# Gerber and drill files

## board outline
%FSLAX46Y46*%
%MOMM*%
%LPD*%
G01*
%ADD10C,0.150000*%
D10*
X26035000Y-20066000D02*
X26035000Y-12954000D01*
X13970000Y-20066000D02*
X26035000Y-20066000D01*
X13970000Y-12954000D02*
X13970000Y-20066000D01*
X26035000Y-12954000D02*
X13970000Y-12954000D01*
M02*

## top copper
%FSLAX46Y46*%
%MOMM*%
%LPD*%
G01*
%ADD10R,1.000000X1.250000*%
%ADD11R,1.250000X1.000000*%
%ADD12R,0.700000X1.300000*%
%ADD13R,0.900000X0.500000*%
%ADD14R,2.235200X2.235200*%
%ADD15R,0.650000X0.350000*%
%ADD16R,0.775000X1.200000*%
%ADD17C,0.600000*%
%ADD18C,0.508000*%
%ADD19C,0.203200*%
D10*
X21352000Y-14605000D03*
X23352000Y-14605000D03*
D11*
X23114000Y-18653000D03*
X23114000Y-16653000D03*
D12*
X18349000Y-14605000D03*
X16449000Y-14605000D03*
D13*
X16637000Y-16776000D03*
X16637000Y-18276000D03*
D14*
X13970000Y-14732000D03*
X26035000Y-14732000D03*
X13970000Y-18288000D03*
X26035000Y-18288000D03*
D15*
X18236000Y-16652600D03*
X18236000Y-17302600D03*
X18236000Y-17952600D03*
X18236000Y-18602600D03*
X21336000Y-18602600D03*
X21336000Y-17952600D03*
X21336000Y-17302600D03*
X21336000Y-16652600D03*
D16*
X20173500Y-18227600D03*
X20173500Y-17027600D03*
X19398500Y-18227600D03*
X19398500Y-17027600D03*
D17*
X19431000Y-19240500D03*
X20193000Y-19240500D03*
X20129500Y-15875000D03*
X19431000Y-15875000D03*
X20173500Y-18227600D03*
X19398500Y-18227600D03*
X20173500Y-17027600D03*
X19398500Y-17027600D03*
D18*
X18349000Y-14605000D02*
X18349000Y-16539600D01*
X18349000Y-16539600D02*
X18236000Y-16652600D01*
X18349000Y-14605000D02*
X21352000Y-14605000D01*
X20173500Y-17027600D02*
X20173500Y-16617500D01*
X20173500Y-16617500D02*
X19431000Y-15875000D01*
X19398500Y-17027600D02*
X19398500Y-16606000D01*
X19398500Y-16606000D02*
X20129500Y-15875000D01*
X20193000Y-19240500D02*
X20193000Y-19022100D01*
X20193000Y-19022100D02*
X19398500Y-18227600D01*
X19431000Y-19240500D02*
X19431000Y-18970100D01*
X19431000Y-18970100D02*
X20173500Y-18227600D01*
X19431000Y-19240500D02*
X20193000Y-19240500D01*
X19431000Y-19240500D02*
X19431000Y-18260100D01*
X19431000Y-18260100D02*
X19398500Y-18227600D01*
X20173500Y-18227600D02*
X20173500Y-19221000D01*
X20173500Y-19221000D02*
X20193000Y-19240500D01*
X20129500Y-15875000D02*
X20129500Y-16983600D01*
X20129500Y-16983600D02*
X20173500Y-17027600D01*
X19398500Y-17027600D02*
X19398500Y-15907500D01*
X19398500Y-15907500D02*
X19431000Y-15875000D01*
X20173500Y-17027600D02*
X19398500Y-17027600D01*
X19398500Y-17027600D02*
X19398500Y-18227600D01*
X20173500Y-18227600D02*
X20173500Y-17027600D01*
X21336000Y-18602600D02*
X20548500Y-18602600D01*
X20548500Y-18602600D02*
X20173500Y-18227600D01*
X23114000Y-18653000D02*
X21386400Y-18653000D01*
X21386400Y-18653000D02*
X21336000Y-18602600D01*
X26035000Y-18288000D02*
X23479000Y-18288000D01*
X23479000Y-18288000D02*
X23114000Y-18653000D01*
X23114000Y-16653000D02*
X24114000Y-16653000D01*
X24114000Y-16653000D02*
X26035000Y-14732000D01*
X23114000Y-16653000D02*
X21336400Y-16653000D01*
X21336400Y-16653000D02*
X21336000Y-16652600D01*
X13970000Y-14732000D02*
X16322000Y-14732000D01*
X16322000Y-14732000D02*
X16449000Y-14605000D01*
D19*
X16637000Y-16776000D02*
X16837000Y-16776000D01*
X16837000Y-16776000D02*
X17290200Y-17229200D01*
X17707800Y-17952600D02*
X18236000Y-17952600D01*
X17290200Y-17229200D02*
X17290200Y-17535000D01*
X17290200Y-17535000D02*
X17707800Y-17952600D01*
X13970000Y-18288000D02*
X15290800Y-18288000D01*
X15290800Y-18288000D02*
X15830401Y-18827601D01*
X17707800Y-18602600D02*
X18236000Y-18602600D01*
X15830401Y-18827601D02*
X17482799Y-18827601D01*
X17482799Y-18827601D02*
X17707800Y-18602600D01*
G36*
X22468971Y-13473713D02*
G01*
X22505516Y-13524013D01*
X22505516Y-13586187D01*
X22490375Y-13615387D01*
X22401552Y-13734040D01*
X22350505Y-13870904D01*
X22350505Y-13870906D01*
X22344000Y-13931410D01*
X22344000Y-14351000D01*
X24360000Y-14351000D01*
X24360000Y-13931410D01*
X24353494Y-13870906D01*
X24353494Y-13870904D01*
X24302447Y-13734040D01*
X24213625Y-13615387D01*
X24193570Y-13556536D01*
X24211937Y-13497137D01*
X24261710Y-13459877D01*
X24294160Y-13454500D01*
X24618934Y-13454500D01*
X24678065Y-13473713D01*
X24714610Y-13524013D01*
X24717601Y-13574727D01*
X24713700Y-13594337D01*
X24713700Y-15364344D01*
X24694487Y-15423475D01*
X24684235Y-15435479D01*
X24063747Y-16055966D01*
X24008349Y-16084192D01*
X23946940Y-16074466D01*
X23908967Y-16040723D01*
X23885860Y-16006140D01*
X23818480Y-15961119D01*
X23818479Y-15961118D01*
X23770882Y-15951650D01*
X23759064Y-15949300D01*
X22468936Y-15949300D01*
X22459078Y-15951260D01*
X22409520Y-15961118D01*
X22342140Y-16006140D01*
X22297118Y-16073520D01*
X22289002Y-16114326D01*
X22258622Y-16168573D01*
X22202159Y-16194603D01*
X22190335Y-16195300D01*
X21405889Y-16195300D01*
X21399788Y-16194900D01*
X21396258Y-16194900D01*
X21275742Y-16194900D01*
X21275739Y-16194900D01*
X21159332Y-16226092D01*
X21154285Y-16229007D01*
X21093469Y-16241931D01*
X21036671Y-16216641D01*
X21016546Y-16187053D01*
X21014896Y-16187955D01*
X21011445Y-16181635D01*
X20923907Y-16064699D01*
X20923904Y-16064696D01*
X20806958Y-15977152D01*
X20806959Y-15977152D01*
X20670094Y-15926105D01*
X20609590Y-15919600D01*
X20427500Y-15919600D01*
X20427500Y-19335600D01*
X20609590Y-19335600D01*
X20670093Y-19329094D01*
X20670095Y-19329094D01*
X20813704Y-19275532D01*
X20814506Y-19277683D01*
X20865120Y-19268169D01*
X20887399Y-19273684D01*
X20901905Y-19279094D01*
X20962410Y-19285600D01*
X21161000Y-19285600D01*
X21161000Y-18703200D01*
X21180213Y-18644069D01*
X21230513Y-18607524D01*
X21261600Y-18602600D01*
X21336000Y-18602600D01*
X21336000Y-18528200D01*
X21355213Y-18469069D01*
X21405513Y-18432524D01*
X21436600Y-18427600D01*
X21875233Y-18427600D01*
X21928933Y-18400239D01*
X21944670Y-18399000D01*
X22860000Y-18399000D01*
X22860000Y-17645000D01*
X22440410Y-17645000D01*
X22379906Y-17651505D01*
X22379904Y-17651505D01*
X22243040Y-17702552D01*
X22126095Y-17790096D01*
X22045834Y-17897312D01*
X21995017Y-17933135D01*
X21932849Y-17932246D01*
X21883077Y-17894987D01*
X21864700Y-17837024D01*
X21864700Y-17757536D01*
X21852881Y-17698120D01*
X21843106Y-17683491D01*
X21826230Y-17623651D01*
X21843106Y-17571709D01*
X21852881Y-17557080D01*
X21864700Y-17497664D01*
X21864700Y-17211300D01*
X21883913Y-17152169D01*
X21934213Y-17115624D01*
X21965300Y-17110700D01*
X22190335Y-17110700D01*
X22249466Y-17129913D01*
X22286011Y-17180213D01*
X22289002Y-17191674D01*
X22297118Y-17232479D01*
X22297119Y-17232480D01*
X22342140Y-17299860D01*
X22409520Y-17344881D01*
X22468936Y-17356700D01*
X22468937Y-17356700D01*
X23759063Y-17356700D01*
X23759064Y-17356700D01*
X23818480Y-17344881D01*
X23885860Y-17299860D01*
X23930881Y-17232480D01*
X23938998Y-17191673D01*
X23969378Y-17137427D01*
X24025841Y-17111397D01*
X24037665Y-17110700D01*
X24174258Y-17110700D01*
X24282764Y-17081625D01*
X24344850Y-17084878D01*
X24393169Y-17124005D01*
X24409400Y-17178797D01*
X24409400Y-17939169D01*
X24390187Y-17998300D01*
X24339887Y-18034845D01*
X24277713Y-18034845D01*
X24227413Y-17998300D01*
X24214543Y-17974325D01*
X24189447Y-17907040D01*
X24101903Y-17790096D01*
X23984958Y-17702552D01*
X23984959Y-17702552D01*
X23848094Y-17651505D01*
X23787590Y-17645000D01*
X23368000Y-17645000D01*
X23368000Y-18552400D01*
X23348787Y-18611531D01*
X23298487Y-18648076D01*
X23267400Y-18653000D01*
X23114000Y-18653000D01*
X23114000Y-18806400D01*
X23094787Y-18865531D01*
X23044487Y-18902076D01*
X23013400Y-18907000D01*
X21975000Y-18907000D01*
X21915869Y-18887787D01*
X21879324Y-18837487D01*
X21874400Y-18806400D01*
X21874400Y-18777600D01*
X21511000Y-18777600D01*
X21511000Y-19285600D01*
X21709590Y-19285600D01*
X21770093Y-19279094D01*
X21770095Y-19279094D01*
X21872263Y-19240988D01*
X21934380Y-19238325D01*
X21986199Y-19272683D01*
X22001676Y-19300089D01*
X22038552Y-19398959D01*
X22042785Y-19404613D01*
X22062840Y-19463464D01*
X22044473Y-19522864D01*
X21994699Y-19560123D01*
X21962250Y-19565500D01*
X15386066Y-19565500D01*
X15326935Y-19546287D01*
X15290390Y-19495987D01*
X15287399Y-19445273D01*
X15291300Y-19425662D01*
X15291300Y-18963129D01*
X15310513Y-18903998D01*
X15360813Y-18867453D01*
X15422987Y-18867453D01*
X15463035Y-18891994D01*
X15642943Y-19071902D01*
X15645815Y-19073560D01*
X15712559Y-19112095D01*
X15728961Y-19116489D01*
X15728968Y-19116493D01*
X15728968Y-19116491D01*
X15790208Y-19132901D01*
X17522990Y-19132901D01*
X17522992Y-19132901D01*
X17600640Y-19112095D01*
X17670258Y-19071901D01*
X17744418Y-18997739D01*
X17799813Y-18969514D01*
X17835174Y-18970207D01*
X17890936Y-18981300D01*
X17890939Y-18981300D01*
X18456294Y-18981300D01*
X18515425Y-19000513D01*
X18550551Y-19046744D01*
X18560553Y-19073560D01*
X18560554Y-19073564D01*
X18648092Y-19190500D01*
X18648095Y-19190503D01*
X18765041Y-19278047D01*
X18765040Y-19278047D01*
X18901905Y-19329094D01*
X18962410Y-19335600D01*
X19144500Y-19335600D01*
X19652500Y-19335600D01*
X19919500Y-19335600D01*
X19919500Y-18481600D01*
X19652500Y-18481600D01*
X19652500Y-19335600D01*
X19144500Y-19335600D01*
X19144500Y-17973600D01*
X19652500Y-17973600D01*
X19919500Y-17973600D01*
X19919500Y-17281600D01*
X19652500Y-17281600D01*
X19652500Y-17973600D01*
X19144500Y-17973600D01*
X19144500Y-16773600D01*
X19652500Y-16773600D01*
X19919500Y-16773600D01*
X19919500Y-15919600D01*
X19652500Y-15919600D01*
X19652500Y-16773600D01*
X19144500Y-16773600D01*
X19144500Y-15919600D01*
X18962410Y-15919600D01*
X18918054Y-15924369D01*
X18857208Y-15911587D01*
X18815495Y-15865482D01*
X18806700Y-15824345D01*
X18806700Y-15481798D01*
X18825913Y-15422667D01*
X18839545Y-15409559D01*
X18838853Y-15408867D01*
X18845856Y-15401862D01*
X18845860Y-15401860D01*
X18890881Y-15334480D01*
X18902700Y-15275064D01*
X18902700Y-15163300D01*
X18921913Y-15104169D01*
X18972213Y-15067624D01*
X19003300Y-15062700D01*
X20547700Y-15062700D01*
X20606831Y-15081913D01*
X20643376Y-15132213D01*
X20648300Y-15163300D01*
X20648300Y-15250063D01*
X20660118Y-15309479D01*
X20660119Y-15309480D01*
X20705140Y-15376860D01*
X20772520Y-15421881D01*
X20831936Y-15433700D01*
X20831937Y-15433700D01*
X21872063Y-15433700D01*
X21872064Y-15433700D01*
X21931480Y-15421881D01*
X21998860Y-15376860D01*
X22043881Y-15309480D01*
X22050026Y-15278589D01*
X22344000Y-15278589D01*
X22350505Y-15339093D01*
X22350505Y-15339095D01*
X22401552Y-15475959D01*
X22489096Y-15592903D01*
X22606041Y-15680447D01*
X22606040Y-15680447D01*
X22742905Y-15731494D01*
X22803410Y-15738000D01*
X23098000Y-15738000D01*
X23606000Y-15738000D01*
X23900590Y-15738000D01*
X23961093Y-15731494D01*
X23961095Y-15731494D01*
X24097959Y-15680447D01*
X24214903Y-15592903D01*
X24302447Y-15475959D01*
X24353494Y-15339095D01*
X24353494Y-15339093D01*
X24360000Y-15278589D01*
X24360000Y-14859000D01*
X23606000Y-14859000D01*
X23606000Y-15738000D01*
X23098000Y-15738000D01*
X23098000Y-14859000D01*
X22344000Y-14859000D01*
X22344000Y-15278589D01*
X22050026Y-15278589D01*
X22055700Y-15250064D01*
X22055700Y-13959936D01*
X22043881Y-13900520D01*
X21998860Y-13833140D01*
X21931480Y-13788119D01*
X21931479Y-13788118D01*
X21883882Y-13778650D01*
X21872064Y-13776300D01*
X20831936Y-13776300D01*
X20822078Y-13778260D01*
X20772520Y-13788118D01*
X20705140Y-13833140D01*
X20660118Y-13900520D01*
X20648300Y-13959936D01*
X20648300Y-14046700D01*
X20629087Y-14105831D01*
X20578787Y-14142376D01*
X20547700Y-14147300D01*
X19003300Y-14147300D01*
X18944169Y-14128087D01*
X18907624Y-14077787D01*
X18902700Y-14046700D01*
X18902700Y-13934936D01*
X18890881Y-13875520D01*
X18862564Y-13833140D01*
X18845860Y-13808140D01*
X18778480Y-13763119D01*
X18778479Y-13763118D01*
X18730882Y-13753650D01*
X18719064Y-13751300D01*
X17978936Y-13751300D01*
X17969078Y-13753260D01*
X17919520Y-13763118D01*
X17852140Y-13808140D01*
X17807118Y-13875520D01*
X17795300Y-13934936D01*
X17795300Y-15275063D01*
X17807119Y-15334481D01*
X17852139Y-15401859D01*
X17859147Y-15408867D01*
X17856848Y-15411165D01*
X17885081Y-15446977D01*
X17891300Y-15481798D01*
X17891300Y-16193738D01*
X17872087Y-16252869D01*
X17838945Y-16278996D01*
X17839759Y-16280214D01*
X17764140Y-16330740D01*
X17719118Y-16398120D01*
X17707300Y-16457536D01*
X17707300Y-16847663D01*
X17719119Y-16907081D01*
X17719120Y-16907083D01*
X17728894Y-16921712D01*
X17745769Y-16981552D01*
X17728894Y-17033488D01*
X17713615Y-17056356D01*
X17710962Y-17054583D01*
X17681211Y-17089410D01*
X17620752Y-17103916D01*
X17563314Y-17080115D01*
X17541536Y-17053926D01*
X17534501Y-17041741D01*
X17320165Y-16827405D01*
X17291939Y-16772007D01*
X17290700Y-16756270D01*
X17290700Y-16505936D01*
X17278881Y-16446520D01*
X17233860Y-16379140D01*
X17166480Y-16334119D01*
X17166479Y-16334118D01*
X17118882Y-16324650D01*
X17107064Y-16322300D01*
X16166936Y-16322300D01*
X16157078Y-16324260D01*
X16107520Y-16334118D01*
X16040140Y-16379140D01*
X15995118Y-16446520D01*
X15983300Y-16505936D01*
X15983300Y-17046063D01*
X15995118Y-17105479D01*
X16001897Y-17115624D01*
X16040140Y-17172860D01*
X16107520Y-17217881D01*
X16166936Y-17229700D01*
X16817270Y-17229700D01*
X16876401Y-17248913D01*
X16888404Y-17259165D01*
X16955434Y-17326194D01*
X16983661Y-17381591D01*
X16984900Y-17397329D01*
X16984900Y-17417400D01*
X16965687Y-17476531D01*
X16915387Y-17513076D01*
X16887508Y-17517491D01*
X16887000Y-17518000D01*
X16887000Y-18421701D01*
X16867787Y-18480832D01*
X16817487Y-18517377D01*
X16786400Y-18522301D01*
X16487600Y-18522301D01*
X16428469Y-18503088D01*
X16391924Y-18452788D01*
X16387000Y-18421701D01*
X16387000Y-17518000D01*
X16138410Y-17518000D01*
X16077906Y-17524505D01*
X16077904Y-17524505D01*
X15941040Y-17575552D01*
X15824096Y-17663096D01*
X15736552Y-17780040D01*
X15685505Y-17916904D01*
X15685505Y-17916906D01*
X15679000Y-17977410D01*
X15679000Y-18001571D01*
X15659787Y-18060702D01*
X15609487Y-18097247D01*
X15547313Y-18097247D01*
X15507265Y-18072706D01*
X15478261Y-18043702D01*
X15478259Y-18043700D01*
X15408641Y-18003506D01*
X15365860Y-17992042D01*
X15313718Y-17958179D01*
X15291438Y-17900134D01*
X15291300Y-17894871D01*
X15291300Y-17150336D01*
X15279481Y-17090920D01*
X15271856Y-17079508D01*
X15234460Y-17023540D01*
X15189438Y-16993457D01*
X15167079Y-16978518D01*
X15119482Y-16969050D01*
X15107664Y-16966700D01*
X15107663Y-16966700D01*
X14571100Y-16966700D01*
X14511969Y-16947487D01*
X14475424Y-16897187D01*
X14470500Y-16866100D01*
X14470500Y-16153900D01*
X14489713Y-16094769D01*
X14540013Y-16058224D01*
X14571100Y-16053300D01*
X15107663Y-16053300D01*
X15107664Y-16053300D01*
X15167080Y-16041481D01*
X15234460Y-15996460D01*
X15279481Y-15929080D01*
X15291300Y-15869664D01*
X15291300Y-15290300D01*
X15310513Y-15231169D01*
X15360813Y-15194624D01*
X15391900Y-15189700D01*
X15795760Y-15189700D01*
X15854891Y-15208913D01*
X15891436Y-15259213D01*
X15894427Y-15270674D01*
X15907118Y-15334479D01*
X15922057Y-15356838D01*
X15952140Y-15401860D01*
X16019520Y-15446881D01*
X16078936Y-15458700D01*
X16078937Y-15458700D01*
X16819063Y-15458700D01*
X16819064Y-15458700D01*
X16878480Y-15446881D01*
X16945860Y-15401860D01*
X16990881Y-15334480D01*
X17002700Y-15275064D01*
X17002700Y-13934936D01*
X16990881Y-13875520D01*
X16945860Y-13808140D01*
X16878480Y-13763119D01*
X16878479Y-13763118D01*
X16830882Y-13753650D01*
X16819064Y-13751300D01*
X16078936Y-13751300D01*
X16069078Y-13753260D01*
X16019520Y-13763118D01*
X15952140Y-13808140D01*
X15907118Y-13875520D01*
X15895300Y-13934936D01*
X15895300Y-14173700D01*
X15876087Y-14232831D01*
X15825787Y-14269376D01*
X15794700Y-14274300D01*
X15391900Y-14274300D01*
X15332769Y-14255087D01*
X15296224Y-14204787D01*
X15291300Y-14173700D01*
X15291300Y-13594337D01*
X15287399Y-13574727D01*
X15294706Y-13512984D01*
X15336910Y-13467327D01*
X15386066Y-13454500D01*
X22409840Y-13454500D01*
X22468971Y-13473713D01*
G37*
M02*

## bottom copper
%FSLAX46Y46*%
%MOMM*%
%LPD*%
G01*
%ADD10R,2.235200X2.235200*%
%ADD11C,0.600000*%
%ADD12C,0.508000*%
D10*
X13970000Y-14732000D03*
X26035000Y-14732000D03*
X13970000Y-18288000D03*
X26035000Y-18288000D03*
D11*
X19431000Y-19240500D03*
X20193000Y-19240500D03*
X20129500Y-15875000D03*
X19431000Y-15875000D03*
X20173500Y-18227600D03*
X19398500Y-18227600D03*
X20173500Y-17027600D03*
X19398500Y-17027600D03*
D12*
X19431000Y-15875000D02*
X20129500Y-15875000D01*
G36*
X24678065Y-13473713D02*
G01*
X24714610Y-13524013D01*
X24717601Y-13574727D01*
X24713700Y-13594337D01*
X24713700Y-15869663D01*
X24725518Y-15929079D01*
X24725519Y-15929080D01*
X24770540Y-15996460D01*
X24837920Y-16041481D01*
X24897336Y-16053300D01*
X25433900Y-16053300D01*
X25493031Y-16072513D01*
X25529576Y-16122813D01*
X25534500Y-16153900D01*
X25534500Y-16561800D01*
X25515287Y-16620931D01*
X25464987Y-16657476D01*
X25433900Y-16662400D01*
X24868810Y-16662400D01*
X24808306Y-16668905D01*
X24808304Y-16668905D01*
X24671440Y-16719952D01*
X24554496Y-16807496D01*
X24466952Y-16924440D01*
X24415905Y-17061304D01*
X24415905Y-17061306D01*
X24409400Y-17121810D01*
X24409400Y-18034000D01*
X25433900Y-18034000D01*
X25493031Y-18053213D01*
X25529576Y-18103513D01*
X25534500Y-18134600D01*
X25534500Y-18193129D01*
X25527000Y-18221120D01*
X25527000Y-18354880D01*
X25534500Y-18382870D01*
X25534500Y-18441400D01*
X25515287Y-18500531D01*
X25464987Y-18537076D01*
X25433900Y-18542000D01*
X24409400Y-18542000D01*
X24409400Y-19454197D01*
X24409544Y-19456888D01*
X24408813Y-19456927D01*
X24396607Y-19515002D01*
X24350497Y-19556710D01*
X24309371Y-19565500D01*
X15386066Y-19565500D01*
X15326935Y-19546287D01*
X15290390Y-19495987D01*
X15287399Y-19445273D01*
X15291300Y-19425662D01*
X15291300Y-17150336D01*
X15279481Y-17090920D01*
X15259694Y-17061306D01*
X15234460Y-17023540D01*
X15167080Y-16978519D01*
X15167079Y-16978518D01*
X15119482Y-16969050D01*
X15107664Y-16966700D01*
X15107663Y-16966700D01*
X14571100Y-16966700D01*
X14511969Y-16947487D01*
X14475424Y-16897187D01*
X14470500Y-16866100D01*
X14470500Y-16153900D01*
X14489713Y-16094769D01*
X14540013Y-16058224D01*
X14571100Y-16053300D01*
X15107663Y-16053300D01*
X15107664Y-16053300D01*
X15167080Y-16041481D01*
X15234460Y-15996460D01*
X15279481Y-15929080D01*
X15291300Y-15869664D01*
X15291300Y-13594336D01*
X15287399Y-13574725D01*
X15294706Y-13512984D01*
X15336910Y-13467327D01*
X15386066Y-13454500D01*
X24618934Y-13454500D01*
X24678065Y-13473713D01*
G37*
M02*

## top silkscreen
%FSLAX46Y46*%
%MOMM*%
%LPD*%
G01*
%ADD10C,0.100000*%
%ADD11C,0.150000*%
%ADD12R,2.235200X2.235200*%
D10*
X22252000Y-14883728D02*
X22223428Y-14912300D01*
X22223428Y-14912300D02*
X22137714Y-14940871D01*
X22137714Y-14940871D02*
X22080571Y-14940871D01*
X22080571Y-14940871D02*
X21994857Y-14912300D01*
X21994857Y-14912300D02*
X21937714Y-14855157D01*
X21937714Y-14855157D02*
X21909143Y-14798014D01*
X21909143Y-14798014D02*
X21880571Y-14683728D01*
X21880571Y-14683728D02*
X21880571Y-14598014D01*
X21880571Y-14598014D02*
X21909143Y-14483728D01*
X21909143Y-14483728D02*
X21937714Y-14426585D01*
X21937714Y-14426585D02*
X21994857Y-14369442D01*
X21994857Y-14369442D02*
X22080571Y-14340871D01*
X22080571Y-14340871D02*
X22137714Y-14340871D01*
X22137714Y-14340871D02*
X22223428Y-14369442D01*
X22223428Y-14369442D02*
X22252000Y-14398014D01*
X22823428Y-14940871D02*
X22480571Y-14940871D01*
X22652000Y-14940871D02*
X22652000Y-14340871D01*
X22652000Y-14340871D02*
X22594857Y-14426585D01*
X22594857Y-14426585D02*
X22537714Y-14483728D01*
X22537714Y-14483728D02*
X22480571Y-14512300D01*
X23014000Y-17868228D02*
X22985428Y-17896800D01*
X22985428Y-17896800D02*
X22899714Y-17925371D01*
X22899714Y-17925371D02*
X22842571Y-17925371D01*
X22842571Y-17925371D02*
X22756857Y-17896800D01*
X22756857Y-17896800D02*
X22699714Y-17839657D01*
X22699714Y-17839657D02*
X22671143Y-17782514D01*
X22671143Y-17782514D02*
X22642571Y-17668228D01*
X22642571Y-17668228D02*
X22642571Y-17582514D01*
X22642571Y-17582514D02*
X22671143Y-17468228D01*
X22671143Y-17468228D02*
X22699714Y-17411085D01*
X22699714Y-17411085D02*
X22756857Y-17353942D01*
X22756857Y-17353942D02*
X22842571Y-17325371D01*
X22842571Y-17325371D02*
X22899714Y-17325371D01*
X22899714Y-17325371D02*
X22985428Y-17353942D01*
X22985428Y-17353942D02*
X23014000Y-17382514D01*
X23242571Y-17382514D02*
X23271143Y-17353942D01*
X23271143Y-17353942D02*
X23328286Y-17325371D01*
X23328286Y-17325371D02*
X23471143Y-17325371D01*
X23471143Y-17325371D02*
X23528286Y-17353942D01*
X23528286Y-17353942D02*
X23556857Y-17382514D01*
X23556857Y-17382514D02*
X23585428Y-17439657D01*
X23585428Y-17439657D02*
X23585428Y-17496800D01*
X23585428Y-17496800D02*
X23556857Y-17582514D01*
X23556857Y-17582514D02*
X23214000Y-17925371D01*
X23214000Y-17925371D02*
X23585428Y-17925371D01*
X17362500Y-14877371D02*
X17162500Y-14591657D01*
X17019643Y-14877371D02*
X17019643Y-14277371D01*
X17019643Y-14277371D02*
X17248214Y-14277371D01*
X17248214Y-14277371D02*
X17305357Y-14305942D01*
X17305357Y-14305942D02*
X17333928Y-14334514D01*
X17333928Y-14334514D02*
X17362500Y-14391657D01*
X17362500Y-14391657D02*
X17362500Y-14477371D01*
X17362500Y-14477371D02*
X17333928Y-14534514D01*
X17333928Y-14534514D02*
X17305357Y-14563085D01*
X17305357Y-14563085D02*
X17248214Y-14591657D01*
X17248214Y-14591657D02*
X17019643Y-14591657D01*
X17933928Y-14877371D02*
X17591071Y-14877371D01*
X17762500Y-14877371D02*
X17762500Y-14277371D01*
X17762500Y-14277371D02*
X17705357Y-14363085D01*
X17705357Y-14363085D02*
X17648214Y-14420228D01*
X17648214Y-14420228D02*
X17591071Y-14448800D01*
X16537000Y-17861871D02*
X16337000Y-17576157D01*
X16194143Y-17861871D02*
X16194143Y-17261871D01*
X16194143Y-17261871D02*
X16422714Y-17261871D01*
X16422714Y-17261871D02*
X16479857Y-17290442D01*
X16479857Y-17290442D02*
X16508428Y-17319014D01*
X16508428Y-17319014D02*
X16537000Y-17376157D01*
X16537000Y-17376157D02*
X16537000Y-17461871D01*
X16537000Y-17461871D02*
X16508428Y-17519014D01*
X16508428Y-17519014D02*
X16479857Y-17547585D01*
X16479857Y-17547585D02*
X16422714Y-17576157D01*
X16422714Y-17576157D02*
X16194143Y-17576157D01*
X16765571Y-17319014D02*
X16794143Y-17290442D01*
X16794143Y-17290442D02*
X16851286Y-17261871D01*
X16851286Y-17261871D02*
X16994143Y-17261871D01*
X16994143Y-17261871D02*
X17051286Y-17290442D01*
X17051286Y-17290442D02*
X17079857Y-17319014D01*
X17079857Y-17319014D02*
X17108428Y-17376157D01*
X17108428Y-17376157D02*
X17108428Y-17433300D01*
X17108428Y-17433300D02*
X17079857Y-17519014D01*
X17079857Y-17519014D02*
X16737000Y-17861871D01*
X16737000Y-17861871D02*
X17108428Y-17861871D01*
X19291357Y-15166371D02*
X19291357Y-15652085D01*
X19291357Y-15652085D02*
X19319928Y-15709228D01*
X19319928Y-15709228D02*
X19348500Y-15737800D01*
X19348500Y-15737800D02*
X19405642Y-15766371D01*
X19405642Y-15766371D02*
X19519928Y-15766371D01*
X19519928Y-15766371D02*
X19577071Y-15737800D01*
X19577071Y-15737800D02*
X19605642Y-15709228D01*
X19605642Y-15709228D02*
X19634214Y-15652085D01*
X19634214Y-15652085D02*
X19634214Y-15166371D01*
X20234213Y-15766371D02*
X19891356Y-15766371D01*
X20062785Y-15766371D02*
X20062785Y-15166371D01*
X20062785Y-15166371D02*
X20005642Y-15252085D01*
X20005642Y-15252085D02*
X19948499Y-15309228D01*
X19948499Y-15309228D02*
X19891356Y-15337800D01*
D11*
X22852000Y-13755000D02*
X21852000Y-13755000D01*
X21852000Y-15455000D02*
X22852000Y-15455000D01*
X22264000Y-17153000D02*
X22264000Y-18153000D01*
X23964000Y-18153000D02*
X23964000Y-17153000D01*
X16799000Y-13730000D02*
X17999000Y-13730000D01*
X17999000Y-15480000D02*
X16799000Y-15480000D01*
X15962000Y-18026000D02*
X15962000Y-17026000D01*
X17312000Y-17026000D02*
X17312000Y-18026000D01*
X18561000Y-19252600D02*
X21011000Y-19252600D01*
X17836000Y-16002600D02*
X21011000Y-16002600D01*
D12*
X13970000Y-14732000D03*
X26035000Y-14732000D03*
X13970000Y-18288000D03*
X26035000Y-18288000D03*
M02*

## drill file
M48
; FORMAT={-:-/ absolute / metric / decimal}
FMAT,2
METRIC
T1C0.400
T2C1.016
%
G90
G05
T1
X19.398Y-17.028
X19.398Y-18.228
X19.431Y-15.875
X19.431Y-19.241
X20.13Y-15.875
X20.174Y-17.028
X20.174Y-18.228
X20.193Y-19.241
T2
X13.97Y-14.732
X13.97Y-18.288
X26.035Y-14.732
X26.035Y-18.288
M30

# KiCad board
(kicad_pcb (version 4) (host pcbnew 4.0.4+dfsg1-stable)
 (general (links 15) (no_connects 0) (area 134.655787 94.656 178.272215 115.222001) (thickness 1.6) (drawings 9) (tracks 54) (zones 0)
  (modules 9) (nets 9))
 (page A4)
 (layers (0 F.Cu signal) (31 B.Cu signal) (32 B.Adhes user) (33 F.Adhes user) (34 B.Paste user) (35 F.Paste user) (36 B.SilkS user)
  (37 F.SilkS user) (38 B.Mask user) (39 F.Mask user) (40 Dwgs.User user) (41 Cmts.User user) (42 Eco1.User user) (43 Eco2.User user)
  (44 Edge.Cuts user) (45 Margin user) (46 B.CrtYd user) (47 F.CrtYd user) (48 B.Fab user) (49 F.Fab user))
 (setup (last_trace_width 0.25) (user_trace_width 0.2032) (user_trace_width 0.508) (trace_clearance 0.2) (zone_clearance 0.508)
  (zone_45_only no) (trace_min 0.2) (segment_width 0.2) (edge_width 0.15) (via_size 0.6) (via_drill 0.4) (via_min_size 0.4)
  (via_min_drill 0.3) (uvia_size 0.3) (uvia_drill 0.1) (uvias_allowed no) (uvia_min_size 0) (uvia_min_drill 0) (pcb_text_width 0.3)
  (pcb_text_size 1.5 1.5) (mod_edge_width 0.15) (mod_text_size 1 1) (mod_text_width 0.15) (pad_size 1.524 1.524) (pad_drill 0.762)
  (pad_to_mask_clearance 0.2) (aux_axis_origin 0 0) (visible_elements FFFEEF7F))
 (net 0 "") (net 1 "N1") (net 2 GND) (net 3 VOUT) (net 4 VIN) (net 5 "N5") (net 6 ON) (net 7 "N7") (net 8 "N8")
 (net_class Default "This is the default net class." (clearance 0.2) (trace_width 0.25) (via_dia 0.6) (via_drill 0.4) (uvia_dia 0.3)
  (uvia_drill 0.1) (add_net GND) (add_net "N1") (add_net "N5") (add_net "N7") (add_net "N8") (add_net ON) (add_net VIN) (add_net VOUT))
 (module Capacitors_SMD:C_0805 (layer F.Cu) (at 22.352 14.605)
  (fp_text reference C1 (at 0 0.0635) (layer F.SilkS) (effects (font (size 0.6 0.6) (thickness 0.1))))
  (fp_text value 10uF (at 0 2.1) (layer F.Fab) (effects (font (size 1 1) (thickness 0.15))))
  (fp_line (start 0.5 -0.85) (end -0.5 -0.85) (layer F.SilkS) (width 0.15))
  (fp_line (start -0.5 0.85) (end 0.5 0.85) (layer F.SilkS) (width 0.15))
  (pad 1 smd rect (at -1 0) (size 1 1.25) (layers F.Cu F.Paste F.Mask) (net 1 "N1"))
  (pad 2 smd rect (at 1 0) (size 1 1.25) (layers F.Cu F.Paste F.Mask) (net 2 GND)))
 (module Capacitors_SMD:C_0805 (layer F.Cu) (at 23.114 17.653 90)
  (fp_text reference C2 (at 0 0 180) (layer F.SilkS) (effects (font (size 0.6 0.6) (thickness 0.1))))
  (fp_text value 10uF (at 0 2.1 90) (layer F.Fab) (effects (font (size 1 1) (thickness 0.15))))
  (fp_line (start 0.5 -0.85) (end -0.5 -0.85) (layer F.SilkS) (width 0.15))
  (fp_line (start -0.5 0.85) (end 0.5 0.85) (layer F.SilkS) (width 0.15))
  (pad 1 smd rect (at -1 0 90) (size 1 1.25) (layers F.Cu F.Paste F.Mask) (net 2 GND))
  (pad 2 smd rect (at 1 0 90) (size 1 1.25) (layers F.Cu F.Paste F.Mask) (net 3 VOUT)))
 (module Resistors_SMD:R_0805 (layer F.Cu) (at 17.399 14.605 180)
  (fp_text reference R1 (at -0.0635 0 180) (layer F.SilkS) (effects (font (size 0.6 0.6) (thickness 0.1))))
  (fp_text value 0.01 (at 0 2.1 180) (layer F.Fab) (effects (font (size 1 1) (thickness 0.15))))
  (fp_line (start 0.6 0.875) (end -0.6 0.875) (layer F.SilkS) (width 0.15))
  (fp_line (start -0.6 -0.875) (end 0.6 -0.875) (layer F.SilkS) (width 0.15))
  (pad 1 smd rect (at -0.95 0 180) (size 0.7 1.3) (layers F.Cu F.Paste F.Mask) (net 1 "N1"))
  (pad 2 smd rect (at 0.95 0 180) (size 0.7 1.3) (layers F.Cu F.Paste F.Mask) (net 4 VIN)))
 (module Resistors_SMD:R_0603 (layer F.Cu) (at 16.637 17.526 270)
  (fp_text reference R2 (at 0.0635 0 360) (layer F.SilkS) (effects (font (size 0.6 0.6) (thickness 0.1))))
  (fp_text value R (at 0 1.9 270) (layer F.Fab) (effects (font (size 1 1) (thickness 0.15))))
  (fp_line (start 0.5 0.675) (end -0.5 0.675) (layer F.SilkS) (width 0.15))
  (fp_line (start -0.5 -0.675) (end 0.5 -0.675) (layer F.SilkS) (width 0.15))
  (pad 1 smd rect (at -0.75 0 270) (size 0.5 0.9) (layers F.Cu F.Paste F.Mask) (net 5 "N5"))
  (pad 2 smd rect (at 0.75 0 270) (size 0.5 0.9) (layers F.Cu F.Paste F.Mask) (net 2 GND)))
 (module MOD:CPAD (layer F.Cu) (at 13.97 14.732)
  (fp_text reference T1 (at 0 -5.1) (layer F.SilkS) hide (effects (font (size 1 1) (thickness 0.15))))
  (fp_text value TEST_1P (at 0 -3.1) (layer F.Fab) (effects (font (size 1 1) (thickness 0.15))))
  (pad 1 thru_hole rect (at 0 0) (size 2.2352 2.2352) (drill 1.016) (layers *.Cu *.Mask F.SilkS) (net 4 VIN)))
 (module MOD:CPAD (layer F.Cu) (at 26.035 14.732)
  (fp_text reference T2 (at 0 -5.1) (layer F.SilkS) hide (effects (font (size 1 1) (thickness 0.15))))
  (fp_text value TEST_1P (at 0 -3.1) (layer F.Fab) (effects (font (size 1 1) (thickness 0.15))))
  (pad 1 thru_hole rect (at 0 0) (size 2.2352 2.2352) (drill 1.016) (layers *.Cu *.Mask F.SilkS) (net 3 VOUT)))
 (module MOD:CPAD (layer F.Cu) (at 13.97 18.288)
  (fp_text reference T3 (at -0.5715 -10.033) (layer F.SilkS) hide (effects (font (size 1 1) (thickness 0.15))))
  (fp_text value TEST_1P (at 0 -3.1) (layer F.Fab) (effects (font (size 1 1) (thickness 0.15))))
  (pad 1 thru_hole rect (at 0 0) (size 2.2352 2.2352) (drill 1.016) (layers *.Cu *.Mask F.SilkS) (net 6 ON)))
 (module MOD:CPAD (layer F.Cu) (at 26.035 18.288)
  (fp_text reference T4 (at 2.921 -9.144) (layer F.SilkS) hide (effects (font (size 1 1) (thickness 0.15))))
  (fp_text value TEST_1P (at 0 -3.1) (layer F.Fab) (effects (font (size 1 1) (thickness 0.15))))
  (pad 1 thru_hole rect (at 0 0) (size 2.2352 2.2352) (drill 1.016) (layers *.Cu *.Mask F.SilkS) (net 2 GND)))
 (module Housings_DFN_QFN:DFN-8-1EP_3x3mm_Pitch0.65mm (layer F.Cu) (at 19.786 17.6276)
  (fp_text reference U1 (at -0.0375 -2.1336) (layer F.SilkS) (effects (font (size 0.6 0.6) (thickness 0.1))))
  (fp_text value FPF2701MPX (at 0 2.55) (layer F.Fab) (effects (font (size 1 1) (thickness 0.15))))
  (fp_line (start -1.225 1.625) (end 1.225 1.625) (layer F.SilkS) (width 0.15))
  (fp_line (start -1.95 -1.625) (end 1.225 -1.625) (layer F.SilkS) (width 0.15))
  (pad 1 smd rect (at -1.55 -0.975) (size 0.65 0.35) (layers F.Cu F.Paste F.Mask) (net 1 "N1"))
  (pad 2 smd rect (at -1.55 -0.325) (size 0.65 0.35) (layers F.Cu F.Paste F.Mask) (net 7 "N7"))
  (pad 3 smd rect (at -1.55 0.325) (size 0.65 0.35) (layers F.Cu F.Paste F.Mask) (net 5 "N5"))
  (pad 4 smd rect (at -1.55 0.975) (size 0.65 0.35) (layers F.Cu F.Paste F.Mask) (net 6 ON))
  (pad 5 smd rect (at 1.55 0.975) (size 0.65 0.35) (layers F.Cu F.Paste F.Mask) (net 2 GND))
  (pad 6 smd rect (at 1.55 0.325) (size 0.65 0.35) (layers F.Cu F.Paste F.Mask))
  (pad 7 smd rect (at 1.55 -0.325) (size 0.65 0.35) (layers F.Cu F.Paste F.Mask) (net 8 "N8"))
  (pad 8 smd rect (at 1.55 -0.975) (size 0.65 0.35) (layers F.Cu F.Paste F.Mask) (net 3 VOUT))
  (pad 9 smd rect (at 0.3875 0.6) (size 0.775 1.2) (layers F.Cu F.Paste F.Mask) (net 2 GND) (solder_paste_margin_ratio -0.2))
  (pad 9 smd rect (at 0.3875 -0.6) (size 0.775 1.2) (layers F.Cu F.Paste F.Mask) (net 2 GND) (solder_paste_margin_ratio -0.2))
  (pad 9 smd rect (at -0.3875 0.6) (size 0.775 1.2) (layers F.Cu F.Paste F.Mask) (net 2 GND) (solder_paste_margin_ratio -0.2))
  (pad 9 smd rect (at -0.3875 -0.6) (size 0.775 1.2) (layers F.Cu F.Paste F.Mask) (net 2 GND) (solder_paste_margin_ratio -0.2)))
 (gr_line (start 26.035 20.066) (end 26.035 12.954) (layer Edge.Cuts) (width 0.15))
 (gr_line (start 13.97 20.066) (end 26.035 20.066) (layer Edge.Cuts) (width 0.15))
 (gr_line (start 13.97 12.954) (end 13.97 20.066) (layer Edge.Cuts) (width 0.15))
 (gr_line (start 26.035 12.954) (end 13.97 12.954) (layer Edge.Cuts) (width 0.15))
 (segment (start 18.349 14.605) (end 18.349 16.5396) (width 0.508) (layer F.Cu) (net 1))
 (segment (start 18.349 16.5396) (end 18.236 16.6526) (width 0.508) (layer F.Cu) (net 1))
 (segment (start 18.349 14.605) (end 21.352 14.605) (width 0.508) (layer F.Cu) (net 1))
 (segment (start 20.1735 17.0276) (end 20.1735 16.6175) (width 0.508) (layer F.Cu) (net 2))
 (segment (start 20.1735 16.6175) (end 19.431 15.875) (width 0.508) (layer F.Cu) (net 2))
 (segment (start 19.3985 17.0276) (end 19.3985 16.606) (width 0.508) (layer F.Cu) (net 2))
 (segment (start 19.3985 16.606) (end 20.1295 15.875) (width 0.508) (layer F.Cu) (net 2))
 (segment (start 20.193 19.2405) (end 20.193 19.0221) (width 0.508) (layer F.Cu) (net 2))
 (segment (start 20.193 19.0221) (end 19.3985 18.2276) (width 0.508) (layer F.Cu) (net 2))
 (segment (start 19.431 19.2405) (end 19.431 18.9701) (width 0.508) (layer F.Cu) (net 2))
 (segment (start 19.431 18.9701) (end 20.1735 18.2276) (width 0.508) (layer F.Cu) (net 2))
 (segment (start 19.431 19.2405) (end 20.193 19.2405) (width 0.508) (layer F.Cu) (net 2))
 (segment (start 19.431 19.2405) (end 19.431 18.2601) (width 0.508) (layer F.Cu) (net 2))
 (segment (start 19.431 18.2601) (end 19.3985 18.2276) (width 0.508) (layer F.Cu) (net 2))
 (via (at 19.431 19.2405) (size 0.6) (drill 0.4) (layers F.Cu B.Cu) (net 2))
 (segment (start 20.1735 18.2276) (end 20.1735 19.221) (width 0.508) (layer F.Cu) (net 2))
 (segment (start 20.1735 19.221) (end 20.193 19.2405) (width 0.508) (layer F.Cu) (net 2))
 (via (at 20.193 19.2405) (size 0.6) (drill 0.4) (layers F.Cu B.Cu) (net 2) (status 1000000))
 (segment (start 20.1295 15.875) (end 20.1295 16.9836) (width 0.508) (layer F.Cu) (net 2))
 (segment (start 20.1295 16.9836) (end 20.1735 17.0276) (width 0.508) (layer F.Cu) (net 2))
 (segment (start 19.431 15.875) (end 20.1295 15.875) (width 0.508) (layer B.Cu) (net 2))
 (via (at 20.1295 15.875) (size 0.6) (drill 0.4) (layers F.Cu B.Cu) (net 2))
 (segment (start 19.3985 17.0276) (end 19.3985 15.9075) (width 0.508) (layer F.Cu) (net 2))
 (segment (start 19.3985 15.9075) (end 19.431 15.875) (width 0.508) (layer F.Cu) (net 2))
 (via (at 19.431 15.875) (size 0.6) (drill 0.4) (layers F.Cu B.Cu) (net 2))
 (segment (start 20.1735 17.0276) (end 19.3985 17.0276) (width 0.508) (layer F.Cu) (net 2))
 (via (at 20.1735 18.2276) (size 0.6) (drill 0.4) (layers F.Cu B.Cu) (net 2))
 (via (at 19.3985 18.2276) (size 0.6) (drill 0.4) (layers F.Cu B.Cu) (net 2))
 (via (at 20.1735 17.0276) (size 0.6) (drill 0.4) (layers F.Cu B.Cu) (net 2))
 (via (at 19.3985 17.0276) (size 0.6) (drill 0.4) (layers F.Cu B.Cu) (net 2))
 (segment (start 19.3985 17.0276) (end 19.3985 18.2276) (width 0.508) (layer F.Cu) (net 2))
 (segment (start 20.1735 18.2276) (end 20.1735 17.0276) (width 0.508) (layer F.Cu) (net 2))
 (segment (start 21.336 18.6026) (end 20.5485 18.6026) (width 0.508) (layer F.Cu) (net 2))
 (segment (start 20.5485 18.6026) (end 20.1735 18.2276) (width 0.508) (layer F.Cu) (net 2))
 (segment (start 23.114 18.653) (end 21.3864 18.653) (width 0.508) (layer F.Cu) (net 2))
 (segment (start 21.3864 18.653) (end 21.336 18.6026) (width 0.508) (layer F.Cu) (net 2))
 (segment (start 26.035 18.288) (end 23.479 18.288) (width 0.508) (layer F.Cu) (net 2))
 (segment (start 23.479 18.288) (end 23.114 18.653) (width 0.508) (layer F.Cu) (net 2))
 (segment (start 23.114 16.653) (end 24.114 16.653) (width 0.508) (layer F.Cu) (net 3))
 (segment (start 24.114 16.653) (end 26.035 14.732) (width 0.508) (layer F.Cu) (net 3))
 (segment (start 23.114 16.653) (end 21.3364 16.653) (width 0.508) (layer F.Cu) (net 3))
 (segment (start 21.3364 16.653) (end 21.336 16.6526) (width 0.508) (layer F.Cu) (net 3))
 (segment (start 13.97 14.732) (end 16.322 14.732) (width 0.508) (layer F.Cu) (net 4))
 (segment (start 16.322 14.732) (end 16.449 14.605) (width 0.508) (layer F.Cu) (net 4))
 (segment (start 16.637 16.776) (end 16.837 16.776) (width 0.2032) (layer F.Cu) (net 5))
 (segment (start 16.837 16.776) (end 17.2902 17.2292) (width 0.2032) (layer F.Cu) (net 5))
 (segment (start 17.7078 17.9526) (end 18.236 17.9526) (width 0.2032) (layer F.Cu) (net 5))
 (segment (start 17.2902 17.2292) (end 17.2902 17.535) (width 0.2032) (layer F.Cu) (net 5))
 (segment (start 17.2902 17.535) (end 17.7078 17.9526) (width 0.2032) (layer F.Cu) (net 5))
 (segment (start 13.97 18.288) (end 15.2908 18.288) (width 0.2032) (layer F.Cu) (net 6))
 (segment (start 15.2908 18.288) (end 15.830401 18.827601) (width 0.2032) (layer F.Cu) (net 6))
 (segment (start 17.7078 18.6026) (end 18.236 18.6026) (width 0.2032) (layer F.Cu) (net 6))
 (segment (start 15.830401 18.827601) (end 17.482799 18.827601) (width 0.2032) (layer F.Cu) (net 6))
 (segment (start 17.482799 18.827601) (end 17.7078 18.6026) (width 0.2032) (layer F.Cu) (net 6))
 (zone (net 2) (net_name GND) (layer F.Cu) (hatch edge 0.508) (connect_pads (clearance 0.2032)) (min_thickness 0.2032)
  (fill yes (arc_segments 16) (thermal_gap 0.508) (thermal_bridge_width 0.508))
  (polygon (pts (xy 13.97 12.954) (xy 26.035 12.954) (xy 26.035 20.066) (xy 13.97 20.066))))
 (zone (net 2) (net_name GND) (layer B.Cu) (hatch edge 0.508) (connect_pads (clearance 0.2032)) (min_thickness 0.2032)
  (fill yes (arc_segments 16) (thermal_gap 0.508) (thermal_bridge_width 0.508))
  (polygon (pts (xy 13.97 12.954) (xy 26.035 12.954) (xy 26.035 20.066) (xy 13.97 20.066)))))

